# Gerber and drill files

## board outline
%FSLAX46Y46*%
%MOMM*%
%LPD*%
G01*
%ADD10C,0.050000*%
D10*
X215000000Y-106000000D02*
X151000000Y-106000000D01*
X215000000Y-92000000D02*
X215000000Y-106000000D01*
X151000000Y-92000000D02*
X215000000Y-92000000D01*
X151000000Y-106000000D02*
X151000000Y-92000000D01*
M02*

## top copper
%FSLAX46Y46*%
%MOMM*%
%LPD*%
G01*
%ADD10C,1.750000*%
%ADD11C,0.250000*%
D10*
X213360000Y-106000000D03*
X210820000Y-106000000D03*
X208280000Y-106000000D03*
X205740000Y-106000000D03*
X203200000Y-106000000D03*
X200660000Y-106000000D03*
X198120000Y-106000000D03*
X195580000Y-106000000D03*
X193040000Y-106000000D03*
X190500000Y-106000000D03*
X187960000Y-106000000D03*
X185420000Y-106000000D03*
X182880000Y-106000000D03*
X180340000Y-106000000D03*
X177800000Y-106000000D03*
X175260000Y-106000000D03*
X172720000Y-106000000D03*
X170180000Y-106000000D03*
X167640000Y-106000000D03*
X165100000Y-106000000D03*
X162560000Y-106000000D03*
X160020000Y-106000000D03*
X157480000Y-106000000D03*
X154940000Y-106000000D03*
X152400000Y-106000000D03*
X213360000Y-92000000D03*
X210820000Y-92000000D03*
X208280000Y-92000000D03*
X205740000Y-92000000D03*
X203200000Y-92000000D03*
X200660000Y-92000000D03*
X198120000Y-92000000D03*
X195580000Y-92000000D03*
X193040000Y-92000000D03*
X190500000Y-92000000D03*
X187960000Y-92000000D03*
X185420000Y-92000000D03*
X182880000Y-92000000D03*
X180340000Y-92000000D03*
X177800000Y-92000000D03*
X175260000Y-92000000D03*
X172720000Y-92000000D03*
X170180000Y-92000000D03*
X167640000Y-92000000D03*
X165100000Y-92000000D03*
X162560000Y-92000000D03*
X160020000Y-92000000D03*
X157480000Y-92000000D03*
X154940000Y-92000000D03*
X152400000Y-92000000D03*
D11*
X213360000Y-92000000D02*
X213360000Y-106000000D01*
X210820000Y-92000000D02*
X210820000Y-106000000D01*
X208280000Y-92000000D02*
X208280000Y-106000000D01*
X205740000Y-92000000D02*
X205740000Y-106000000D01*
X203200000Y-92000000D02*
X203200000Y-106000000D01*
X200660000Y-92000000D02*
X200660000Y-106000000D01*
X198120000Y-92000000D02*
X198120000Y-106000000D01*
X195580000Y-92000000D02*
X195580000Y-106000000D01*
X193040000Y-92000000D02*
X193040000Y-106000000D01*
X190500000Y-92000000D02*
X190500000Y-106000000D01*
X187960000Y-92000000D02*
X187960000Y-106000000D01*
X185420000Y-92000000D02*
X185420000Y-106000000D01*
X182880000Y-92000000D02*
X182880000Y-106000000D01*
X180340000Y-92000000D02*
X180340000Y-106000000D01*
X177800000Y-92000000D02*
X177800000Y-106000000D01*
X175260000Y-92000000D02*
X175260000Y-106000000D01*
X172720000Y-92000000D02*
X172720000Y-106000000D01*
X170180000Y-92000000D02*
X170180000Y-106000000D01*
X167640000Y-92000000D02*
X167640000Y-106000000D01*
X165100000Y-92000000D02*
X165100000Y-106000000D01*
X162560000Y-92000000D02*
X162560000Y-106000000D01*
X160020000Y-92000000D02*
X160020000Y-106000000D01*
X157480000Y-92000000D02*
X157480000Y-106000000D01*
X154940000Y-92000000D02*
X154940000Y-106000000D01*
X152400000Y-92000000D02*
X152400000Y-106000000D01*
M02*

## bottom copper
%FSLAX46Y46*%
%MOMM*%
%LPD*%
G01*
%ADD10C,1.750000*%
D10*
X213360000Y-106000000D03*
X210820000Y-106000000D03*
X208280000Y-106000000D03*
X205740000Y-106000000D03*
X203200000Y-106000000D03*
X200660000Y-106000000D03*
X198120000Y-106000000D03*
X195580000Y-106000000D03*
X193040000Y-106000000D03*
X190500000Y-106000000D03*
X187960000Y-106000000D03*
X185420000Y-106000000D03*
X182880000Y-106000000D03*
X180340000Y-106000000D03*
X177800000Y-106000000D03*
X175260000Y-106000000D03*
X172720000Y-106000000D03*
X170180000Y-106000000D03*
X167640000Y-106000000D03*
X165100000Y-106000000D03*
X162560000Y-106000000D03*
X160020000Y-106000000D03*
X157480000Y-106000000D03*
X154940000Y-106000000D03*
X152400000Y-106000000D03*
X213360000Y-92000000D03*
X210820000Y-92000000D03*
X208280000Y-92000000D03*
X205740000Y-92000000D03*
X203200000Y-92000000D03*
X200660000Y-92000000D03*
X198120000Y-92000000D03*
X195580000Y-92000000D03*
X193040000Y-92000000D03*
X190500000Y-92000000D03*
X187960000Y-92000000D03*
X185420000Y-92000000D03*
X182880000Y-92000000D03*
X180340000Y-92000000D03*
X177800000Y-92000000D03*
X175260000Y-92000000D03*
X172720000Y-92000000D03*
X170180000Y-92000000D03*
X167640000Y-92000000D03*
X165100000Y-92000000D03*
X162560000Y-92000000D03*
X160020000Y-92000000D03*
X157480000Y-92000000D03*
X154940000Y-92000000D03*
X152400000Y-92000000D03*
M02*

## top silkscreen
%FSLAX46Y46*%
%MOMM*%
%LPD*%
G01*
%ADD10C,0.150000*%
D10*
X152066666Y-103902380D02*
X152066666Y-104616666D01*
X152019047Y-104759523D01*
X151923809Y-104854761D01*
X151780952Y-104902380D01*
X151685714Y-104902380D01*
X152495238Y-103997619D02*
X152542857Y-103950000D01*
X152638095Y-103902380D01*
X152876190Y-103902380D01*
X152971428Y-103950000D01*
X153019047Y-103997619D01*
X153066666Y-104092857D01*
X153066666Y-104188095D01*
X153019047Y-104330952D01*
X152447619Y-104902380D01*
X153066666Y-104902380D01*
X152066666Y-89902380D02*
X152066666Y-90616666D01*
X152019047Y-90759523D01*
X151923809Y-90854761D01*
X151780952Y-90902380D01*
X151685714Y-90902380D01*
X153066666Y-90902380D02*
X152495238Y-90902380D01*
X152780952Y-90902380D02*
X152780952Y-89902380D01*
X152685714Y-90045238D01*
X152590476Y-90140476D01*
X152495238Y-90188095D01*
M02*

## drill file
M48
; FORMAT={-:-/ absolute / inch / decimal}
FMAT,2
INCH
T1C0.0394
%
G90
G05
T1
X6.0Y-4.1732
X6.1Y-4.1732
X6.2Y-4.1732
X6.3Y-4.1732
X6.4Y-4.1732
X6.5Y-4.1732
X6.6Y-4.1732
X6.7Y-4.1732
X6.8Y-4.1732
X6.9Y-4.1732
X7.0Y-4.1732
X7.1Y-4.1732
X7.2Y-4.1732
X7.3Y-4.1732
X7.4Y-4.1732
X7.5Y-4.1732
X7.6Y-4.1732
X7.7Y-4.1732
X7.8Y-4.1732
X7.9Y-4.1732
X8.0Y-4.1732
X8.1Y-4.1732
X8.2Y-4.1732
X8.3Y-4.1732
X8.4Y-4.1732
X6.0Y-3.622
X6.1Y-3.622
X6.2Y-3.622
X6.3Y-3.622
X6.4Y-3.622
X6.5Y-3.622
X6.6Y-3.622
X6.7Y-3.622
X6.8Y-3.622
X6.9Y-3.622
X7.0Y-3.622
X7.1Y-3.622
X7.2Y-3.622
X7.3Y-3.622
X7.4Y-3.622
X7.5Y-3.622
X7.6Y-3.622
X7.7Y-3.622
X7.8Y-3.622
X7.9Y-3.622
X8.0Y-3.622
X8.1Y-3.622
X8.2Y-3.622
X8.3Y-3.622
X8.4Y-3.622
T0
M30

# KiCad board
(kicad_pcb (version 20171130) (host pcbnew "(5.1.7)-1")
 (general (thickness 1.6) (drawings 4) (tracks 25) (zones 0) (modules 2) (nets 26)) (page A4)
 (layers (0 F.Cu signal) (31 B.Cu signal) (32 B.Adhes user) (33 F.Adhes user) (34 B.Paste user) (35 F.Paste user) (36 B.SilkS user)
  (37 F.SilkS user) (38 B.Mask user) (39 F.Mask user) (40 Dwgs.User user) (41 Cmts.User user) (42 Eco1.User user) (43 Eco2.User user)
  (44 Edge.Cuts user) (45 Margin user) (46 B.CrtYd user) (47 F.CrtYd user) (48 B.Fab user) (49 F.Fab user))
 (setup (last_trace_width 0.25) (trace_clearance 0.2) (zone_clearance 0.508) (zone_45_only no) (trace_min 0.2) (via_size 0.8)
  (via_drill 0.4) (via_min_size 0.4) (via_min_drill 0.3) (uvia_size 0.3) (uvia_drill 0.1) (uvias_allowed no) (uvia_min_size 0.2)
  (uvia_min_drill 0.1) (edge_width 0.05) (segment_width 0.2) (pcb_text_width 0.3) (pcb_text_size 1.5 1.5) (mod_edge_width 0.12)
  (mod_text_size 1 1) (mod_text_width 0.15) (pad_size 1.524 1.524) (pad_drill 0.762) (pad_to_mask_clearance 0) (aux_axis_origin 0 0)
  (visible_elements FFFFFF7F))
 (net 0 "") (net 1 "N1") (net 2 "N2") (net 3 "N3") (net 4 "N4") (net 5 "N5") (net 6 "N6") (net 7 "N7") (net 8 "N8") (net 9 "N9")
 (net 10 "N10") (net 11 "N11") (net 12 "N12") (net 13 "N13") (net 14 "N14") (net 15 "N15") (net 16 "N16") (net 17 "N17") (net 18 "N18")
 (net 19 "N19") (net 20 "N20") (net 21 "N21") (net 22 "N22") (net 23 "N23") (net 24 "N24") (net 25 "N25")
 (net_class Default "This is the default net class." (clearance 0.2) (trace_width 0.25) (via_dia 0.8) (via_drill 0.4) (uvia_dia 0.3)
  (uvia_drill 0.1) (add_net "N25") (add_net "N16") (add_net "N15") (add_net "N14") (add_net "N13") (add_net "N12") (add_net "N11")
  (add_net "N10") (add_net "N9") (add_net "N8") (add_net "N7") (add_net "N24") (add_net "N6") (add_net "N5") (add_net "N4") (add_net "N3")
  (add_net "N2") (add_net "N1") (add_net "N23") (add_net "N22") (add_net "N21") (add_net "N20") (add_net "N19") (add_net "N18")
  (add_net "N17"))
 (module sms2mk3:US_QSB (layer F.Cu) (at 152.4 106)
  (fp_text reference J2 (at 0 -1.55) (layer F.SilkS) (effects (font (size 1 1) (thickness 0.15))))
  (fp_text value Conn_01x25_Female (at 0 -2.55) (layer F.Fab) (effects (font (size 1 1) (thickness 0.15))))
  (pad 25 thru_hole circle (at 60.96 0) (size 1.75 1.75) (drill 1) (layers *.Cu *.Mask) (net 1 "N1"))
  (pad 24 thru_hole circle (at 58.42 0) (size 1.75 1.75) (drill 1) (layers *.Cu *.Mask) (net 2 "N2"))
  (pad 23 thru_hole circle (at 55.88 0) (size 1.75 1.75) (drill 1) (layers *.Cu *.Mask) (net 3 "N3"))
  (pad 22 thru_hole circle (at 53.34 0) (size 1.75 1.75) (drill 1) (layers *.Cu *.Mask) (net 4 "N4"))
  (pad 21 thru_hole circle (at 50.8 0) (size 1.75 1.75) (drill 1) (layers *.Cu *.Mask) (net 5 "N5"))
  (pad 20 thru_hole circle (at 48.26 0) (size 1.75 1.75) (drill 1) (layers *.Cu *.Mask) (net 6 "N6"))
  (pad 19 thru_hole circle (at 45.72 0) (size 1.75 1.75) (drill 1) (layers *.Cu *.Mask) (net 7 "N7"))
  (pad 18 thru_hole circle (at 43.18 0) (size 1.75 1.75) (drill 1) (layers *.Cu *.Mask) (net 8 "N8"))
  (pad 17 thru_hole circle (at 40.64 0) (size 1.75 1.75) (drill 1) (layers *.Cu *.Mask) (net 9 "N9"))
  (pad 16 thru_hole circle (at 38.1 0) (size 1.75 1.75) (drill 1) (layers *.Cu *.Mask) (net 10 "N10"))
  (pad 15 thru_hole circle (at 35.56 0) (size 1.75 1.75) (drill 1) (layers *.Cu *.Mask) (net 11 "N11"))
  (pad 14 thru_hole circle (at 33.02 0) (size 1.75 1.75) (drill 1) (layers *.Cu *.Mask) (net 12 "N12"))
  (pad 13 thru_hole circle (at 30.48 0) (size 1.75 1.75) (drill 1) (layers *.Cu *.Mask) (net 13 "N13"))
  (pad 12 thru_hole circle (at 27.94 0) (size 1.75 1.75) (drill 1) (layers *.Cu *.Mask) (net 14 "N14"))
  (pad 11 thru_hole circle (at 25.4 0) (size 1.75 1.75) (drill 1) (layers *.Cu *.Mask) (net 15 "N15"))
  (pad 10 thru_hole circle (at 22.86 0) (size 1.75 1.75) (drill 1) (layers *.Cu *.Mask) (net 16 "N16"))
  (pad 9 thru_hole circle (at 20.32 0) (size 1.75 1.75) (drill 1) (layers *.Cu *.Mask) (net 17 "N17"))
  (pad 8 thru_hole circle (at 17.78 0) (size 1.75 1.75) (drill 1) (layers *.Cu *.Mask) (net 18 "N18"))
  (pad 7 thru_hole circle (at 15.24 0) (size 1.75 1.75) (drill 1) (layers *.Cu *.Mask) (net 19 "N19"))
  (pad 6 thru_hole circle (at 12.7 0) (size 1.75 1.75) (drill 1) (layers *.Cu *.Mask) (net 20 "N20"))
  (pad 5 thru_hole circle (at 10.16 0) (size 1.75 1.75) (drill 1) (layers *.Cu *.Mask) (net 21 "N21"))
  (pad 4 thru_hole circle (at 7.62 0) (size 1.75 1.75) (drill 1) (layers *.Cu *.Mask) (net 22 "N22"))
  (pad 3 thru_hole circle (at 5.08 0) (size 1.75 1.75) (drill 1) (layers *.Cu *.Mask) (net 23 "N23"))
  (pad 2 thru_hole circle (at 2.54 0) (size 1.75 1.75) (drill 1) (layers *.Cu *.Mask) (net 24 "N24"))
  (pad 1 thru_hole circle (at 0 0) (size 1.75 1.75) (drill 1) (layers *.Cu *.Mask) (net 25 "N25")))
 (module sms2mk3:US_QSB (layer F.Cu) (at 152.4 92)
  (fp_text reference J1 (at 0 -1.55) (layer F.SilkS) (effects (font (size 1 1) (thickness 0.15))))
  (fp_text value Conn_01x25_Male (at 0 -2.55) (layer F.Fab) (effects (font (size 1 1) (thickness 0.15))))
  (pad 25 thru_hole circle (at 60.96 0) (size 1.75 1.75) (drill 1) (layers *.Cu *.Mask) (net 1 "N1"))
  (pad 24 thru_hole circle (at 58.42 0) (size 1.75 1.75) (drill 1) (layers *.Cu *.Mask) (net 2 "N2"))
  (pad 23 thru_hole circle (at 55.88 0) (size 1.75 1.75) (drill 1) (layers *.Cu *.Mask) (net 3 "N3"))
  (pad 22 thru_hole circle (at 53.34 0) (size 1.75 1.75) (drill 1) (layers *.Cu *.Mask) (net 4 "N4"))
  (pad 21 thru_hole circle (at 50.8 0) (size 1.75 1.75) (drill 1) (layers *.Cu *.Mask) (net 5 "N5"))
  (pad 20 thru_hole circle (at 48.26 0) (size 1.75 1.75) (drill 1) (layers *.Cu *.Mask) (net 6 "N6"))
  (pad 19 thru_hole circle (at 45.72 0) (size 1.75 1.75) (drill 1) (layers *.Cu *.Mask) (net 7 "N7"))
  (pad 18 thru_hole circle (at 43.18 0) (size 1.75 1.75) (drill 1) (layers *.Cu *.Mask) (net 8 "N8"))
  (pad 17 thru_hole circle (at 40.64 0) (size 1.75 1.75) (drill 1) (layers *.Cu *.Mask) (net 9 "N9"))
  (pad 16 thru_hole circle (at 38.1 0) (size 1.75 1.75) (drill 1) (layers *.Cu *.Mask) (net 10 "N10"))
  (pad 15 thru_hole circle (at 35.56 0) (size 1.75 1.75) (drill 1) (layers *.Cu *.Mask) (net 11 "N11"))
  (pad 14 thru_hole circle (at 33.02 0) (size 1.75 1.75) (drill 1) (layers *.Cu *.Mask) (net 12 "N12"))
  (pad 13 thru_hole circle (at 30.48 0) (size 1.75 1.75) (drill 1) (layers *.Cu *.Mask) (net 13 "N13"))
  (pad 12 thru_hole circle (at 27.94 0) (size 1.75 1.75) (drill 1) (layers *.Cu *.Mask) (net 14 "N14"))
  (pad 11 thru_hole circle (at 25.4 0) (size 1.75 1.75) (drill 1) (layers *.Cu *.Mask) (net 15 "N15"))
  (pad 10 thru_hole circle (at 22.86 0) (size 1.75 1.75) (drill 1) (layers *.Cu *.Mask) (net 16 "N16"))
  (pad 9 thru_hole circle (at 20.32 0) (size 1.75 1.75) (drill 1) (layers *.Cu *.Mask) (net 17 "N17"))
  (pad 8 thru_hole circle (at 17.78 0) (size 1.75 1.75) (drill 1) (layers *.Cu *.Mask) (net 18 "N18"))
  (pad 7 thru_hole circle (at 15.24 0) (size 1.75 1.75) (drill 1) (layers *.Cu *.Mask) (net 19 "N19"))
  (pad 6 thru_hole circle (at 12.7 0) (size 1.75 1.75) (drill 1) (layers *.Cu *.Mask) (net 20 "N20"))
  (pad 5 thru_hole circle (at 10.16 0) (size 1.75 1.75) (drill 1) (layers *.Cu *.Mask) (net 21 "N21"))
  (pad 4 thru_hole circle (at 7.62 0) (size 1.75 1.75) (drill 1) (layers *.Cu *.Mask) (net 22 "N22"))
  (pad 3 thru_hole circle (at 5.08 0) (size 1.75 1.75) (drill 1) (layers *.Cu *.Mask) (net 23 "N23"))
  (pad 2 thru_hole circle (at 2.54 0) (size 1.75 1.75) (drill 1) (layers *.Cu *.Mask) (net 24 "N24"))
  (pad 1 thru_hole circle (at 0 0) (size 1.75 1.75) (drill 1) (layers *.Cu *.Mask) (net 25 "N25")))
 (gr_line (start 215 106) (end 151 106) (layer Edge.Cuts) (width 0.05))
 (gr_line (start 215 92) (end 215 106) (layer Edge.Cuts) (width 0.05))
 (gr_line (start 151 92) (end 215 92) (layer Edge.Cuts) (width 0.05))
 (gr_line (start 151 106) (end 151 92) (layer Edge.Cuts) (width 0.05))
 (segment (start 213.36 92) (end 213.36 106) (width 0.25) (layer F.Cu) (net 1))
 (segment (start 210.82 92) (end 210.82 106) (width 0.25) (layer F.Cu) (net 2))
 (segment (start 208.28 92) (end 208.28 106) (width 0.25) (layer F.Cu) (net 3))
 (segment (start 205.74 92) (end 205.74 106) (width 0.25) (layer F.Cu) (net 4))
 (segment (start 203.2 92) (end 203.2 106) (width 0.25) (layer F.Cu) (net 5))
 (segment (start 200.66 92) (end 200.66 106) (width 0.25) (layer F.Cu) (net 6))
 (segment (start 198.12 92) (end 198.12 106) (width 0.25) (layer F.Cu) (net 7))
 (segment (start 195.58 92) (end 195.58 106) (width 0.25) (layer F.Cu) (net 8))
 (segment (start 193.04 92) (end 193.04 106) (width 0.25) (layer F.Cu) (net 9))
 (segment (start 190.5 92) (end 190.5 106) (width 0.25) (layer F.Cu) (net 10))
 (segment (start 187.96 92) (end 187.96 106) (width 0.25) (layer F.Cu) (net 11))
 (segment (start 185.42 92) (end 185.42 106) (width 0.25) (layer F.Cu) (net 12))
 (segment (start 182.88 92) (end 182.88 106) (width 0.25) (layer F.Cu) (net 13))
 (segment (start 180.34 92) (end 180.34 106) (width 0.25) (layer F.Cu) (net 14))
 (segment (start 177.8 92) (end 177.8 106) (width 0.25) (layer F.Cu) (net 15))
 (segment (start 175.26 92) (end 175.26 106) (width 0.25) (layer F.Cu) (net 16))
 (segment (start 172.72 92) (end 172.72 106) (width 0.25) (layer F.Cu) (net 17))
 (segment (start 170.18 92) (end 170.18 106) (width 0.25) (layer F.Cu) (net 18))
 (segment (start 167.64 92) (end 167.64 106) (width 0.25) (layer F.Cu) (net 19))
 (segment (start 165.1 92) (end 165.1 106) (width 0.25) (layer F.Cu) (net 20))
 (segment (start 162.56 92) (end 162.56 106) (width 0.25) (layer F.Cu) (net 21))
 (segment (start 160.02 92) (end 160.02 106) (width 0.25) (layer F.Cu) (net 22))
 (segment (start 157.48 92) (end 157.48 106) (width 0.25) (layer F.Cu) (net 23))
 (segment (start 154.94 92) (end 154.94 106) (width 0.25) (layer F.Cu) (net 24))
 (segment (start 152.4 92) (end 152.4 106) (width 0.25) (layer F.Cu) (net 25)))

